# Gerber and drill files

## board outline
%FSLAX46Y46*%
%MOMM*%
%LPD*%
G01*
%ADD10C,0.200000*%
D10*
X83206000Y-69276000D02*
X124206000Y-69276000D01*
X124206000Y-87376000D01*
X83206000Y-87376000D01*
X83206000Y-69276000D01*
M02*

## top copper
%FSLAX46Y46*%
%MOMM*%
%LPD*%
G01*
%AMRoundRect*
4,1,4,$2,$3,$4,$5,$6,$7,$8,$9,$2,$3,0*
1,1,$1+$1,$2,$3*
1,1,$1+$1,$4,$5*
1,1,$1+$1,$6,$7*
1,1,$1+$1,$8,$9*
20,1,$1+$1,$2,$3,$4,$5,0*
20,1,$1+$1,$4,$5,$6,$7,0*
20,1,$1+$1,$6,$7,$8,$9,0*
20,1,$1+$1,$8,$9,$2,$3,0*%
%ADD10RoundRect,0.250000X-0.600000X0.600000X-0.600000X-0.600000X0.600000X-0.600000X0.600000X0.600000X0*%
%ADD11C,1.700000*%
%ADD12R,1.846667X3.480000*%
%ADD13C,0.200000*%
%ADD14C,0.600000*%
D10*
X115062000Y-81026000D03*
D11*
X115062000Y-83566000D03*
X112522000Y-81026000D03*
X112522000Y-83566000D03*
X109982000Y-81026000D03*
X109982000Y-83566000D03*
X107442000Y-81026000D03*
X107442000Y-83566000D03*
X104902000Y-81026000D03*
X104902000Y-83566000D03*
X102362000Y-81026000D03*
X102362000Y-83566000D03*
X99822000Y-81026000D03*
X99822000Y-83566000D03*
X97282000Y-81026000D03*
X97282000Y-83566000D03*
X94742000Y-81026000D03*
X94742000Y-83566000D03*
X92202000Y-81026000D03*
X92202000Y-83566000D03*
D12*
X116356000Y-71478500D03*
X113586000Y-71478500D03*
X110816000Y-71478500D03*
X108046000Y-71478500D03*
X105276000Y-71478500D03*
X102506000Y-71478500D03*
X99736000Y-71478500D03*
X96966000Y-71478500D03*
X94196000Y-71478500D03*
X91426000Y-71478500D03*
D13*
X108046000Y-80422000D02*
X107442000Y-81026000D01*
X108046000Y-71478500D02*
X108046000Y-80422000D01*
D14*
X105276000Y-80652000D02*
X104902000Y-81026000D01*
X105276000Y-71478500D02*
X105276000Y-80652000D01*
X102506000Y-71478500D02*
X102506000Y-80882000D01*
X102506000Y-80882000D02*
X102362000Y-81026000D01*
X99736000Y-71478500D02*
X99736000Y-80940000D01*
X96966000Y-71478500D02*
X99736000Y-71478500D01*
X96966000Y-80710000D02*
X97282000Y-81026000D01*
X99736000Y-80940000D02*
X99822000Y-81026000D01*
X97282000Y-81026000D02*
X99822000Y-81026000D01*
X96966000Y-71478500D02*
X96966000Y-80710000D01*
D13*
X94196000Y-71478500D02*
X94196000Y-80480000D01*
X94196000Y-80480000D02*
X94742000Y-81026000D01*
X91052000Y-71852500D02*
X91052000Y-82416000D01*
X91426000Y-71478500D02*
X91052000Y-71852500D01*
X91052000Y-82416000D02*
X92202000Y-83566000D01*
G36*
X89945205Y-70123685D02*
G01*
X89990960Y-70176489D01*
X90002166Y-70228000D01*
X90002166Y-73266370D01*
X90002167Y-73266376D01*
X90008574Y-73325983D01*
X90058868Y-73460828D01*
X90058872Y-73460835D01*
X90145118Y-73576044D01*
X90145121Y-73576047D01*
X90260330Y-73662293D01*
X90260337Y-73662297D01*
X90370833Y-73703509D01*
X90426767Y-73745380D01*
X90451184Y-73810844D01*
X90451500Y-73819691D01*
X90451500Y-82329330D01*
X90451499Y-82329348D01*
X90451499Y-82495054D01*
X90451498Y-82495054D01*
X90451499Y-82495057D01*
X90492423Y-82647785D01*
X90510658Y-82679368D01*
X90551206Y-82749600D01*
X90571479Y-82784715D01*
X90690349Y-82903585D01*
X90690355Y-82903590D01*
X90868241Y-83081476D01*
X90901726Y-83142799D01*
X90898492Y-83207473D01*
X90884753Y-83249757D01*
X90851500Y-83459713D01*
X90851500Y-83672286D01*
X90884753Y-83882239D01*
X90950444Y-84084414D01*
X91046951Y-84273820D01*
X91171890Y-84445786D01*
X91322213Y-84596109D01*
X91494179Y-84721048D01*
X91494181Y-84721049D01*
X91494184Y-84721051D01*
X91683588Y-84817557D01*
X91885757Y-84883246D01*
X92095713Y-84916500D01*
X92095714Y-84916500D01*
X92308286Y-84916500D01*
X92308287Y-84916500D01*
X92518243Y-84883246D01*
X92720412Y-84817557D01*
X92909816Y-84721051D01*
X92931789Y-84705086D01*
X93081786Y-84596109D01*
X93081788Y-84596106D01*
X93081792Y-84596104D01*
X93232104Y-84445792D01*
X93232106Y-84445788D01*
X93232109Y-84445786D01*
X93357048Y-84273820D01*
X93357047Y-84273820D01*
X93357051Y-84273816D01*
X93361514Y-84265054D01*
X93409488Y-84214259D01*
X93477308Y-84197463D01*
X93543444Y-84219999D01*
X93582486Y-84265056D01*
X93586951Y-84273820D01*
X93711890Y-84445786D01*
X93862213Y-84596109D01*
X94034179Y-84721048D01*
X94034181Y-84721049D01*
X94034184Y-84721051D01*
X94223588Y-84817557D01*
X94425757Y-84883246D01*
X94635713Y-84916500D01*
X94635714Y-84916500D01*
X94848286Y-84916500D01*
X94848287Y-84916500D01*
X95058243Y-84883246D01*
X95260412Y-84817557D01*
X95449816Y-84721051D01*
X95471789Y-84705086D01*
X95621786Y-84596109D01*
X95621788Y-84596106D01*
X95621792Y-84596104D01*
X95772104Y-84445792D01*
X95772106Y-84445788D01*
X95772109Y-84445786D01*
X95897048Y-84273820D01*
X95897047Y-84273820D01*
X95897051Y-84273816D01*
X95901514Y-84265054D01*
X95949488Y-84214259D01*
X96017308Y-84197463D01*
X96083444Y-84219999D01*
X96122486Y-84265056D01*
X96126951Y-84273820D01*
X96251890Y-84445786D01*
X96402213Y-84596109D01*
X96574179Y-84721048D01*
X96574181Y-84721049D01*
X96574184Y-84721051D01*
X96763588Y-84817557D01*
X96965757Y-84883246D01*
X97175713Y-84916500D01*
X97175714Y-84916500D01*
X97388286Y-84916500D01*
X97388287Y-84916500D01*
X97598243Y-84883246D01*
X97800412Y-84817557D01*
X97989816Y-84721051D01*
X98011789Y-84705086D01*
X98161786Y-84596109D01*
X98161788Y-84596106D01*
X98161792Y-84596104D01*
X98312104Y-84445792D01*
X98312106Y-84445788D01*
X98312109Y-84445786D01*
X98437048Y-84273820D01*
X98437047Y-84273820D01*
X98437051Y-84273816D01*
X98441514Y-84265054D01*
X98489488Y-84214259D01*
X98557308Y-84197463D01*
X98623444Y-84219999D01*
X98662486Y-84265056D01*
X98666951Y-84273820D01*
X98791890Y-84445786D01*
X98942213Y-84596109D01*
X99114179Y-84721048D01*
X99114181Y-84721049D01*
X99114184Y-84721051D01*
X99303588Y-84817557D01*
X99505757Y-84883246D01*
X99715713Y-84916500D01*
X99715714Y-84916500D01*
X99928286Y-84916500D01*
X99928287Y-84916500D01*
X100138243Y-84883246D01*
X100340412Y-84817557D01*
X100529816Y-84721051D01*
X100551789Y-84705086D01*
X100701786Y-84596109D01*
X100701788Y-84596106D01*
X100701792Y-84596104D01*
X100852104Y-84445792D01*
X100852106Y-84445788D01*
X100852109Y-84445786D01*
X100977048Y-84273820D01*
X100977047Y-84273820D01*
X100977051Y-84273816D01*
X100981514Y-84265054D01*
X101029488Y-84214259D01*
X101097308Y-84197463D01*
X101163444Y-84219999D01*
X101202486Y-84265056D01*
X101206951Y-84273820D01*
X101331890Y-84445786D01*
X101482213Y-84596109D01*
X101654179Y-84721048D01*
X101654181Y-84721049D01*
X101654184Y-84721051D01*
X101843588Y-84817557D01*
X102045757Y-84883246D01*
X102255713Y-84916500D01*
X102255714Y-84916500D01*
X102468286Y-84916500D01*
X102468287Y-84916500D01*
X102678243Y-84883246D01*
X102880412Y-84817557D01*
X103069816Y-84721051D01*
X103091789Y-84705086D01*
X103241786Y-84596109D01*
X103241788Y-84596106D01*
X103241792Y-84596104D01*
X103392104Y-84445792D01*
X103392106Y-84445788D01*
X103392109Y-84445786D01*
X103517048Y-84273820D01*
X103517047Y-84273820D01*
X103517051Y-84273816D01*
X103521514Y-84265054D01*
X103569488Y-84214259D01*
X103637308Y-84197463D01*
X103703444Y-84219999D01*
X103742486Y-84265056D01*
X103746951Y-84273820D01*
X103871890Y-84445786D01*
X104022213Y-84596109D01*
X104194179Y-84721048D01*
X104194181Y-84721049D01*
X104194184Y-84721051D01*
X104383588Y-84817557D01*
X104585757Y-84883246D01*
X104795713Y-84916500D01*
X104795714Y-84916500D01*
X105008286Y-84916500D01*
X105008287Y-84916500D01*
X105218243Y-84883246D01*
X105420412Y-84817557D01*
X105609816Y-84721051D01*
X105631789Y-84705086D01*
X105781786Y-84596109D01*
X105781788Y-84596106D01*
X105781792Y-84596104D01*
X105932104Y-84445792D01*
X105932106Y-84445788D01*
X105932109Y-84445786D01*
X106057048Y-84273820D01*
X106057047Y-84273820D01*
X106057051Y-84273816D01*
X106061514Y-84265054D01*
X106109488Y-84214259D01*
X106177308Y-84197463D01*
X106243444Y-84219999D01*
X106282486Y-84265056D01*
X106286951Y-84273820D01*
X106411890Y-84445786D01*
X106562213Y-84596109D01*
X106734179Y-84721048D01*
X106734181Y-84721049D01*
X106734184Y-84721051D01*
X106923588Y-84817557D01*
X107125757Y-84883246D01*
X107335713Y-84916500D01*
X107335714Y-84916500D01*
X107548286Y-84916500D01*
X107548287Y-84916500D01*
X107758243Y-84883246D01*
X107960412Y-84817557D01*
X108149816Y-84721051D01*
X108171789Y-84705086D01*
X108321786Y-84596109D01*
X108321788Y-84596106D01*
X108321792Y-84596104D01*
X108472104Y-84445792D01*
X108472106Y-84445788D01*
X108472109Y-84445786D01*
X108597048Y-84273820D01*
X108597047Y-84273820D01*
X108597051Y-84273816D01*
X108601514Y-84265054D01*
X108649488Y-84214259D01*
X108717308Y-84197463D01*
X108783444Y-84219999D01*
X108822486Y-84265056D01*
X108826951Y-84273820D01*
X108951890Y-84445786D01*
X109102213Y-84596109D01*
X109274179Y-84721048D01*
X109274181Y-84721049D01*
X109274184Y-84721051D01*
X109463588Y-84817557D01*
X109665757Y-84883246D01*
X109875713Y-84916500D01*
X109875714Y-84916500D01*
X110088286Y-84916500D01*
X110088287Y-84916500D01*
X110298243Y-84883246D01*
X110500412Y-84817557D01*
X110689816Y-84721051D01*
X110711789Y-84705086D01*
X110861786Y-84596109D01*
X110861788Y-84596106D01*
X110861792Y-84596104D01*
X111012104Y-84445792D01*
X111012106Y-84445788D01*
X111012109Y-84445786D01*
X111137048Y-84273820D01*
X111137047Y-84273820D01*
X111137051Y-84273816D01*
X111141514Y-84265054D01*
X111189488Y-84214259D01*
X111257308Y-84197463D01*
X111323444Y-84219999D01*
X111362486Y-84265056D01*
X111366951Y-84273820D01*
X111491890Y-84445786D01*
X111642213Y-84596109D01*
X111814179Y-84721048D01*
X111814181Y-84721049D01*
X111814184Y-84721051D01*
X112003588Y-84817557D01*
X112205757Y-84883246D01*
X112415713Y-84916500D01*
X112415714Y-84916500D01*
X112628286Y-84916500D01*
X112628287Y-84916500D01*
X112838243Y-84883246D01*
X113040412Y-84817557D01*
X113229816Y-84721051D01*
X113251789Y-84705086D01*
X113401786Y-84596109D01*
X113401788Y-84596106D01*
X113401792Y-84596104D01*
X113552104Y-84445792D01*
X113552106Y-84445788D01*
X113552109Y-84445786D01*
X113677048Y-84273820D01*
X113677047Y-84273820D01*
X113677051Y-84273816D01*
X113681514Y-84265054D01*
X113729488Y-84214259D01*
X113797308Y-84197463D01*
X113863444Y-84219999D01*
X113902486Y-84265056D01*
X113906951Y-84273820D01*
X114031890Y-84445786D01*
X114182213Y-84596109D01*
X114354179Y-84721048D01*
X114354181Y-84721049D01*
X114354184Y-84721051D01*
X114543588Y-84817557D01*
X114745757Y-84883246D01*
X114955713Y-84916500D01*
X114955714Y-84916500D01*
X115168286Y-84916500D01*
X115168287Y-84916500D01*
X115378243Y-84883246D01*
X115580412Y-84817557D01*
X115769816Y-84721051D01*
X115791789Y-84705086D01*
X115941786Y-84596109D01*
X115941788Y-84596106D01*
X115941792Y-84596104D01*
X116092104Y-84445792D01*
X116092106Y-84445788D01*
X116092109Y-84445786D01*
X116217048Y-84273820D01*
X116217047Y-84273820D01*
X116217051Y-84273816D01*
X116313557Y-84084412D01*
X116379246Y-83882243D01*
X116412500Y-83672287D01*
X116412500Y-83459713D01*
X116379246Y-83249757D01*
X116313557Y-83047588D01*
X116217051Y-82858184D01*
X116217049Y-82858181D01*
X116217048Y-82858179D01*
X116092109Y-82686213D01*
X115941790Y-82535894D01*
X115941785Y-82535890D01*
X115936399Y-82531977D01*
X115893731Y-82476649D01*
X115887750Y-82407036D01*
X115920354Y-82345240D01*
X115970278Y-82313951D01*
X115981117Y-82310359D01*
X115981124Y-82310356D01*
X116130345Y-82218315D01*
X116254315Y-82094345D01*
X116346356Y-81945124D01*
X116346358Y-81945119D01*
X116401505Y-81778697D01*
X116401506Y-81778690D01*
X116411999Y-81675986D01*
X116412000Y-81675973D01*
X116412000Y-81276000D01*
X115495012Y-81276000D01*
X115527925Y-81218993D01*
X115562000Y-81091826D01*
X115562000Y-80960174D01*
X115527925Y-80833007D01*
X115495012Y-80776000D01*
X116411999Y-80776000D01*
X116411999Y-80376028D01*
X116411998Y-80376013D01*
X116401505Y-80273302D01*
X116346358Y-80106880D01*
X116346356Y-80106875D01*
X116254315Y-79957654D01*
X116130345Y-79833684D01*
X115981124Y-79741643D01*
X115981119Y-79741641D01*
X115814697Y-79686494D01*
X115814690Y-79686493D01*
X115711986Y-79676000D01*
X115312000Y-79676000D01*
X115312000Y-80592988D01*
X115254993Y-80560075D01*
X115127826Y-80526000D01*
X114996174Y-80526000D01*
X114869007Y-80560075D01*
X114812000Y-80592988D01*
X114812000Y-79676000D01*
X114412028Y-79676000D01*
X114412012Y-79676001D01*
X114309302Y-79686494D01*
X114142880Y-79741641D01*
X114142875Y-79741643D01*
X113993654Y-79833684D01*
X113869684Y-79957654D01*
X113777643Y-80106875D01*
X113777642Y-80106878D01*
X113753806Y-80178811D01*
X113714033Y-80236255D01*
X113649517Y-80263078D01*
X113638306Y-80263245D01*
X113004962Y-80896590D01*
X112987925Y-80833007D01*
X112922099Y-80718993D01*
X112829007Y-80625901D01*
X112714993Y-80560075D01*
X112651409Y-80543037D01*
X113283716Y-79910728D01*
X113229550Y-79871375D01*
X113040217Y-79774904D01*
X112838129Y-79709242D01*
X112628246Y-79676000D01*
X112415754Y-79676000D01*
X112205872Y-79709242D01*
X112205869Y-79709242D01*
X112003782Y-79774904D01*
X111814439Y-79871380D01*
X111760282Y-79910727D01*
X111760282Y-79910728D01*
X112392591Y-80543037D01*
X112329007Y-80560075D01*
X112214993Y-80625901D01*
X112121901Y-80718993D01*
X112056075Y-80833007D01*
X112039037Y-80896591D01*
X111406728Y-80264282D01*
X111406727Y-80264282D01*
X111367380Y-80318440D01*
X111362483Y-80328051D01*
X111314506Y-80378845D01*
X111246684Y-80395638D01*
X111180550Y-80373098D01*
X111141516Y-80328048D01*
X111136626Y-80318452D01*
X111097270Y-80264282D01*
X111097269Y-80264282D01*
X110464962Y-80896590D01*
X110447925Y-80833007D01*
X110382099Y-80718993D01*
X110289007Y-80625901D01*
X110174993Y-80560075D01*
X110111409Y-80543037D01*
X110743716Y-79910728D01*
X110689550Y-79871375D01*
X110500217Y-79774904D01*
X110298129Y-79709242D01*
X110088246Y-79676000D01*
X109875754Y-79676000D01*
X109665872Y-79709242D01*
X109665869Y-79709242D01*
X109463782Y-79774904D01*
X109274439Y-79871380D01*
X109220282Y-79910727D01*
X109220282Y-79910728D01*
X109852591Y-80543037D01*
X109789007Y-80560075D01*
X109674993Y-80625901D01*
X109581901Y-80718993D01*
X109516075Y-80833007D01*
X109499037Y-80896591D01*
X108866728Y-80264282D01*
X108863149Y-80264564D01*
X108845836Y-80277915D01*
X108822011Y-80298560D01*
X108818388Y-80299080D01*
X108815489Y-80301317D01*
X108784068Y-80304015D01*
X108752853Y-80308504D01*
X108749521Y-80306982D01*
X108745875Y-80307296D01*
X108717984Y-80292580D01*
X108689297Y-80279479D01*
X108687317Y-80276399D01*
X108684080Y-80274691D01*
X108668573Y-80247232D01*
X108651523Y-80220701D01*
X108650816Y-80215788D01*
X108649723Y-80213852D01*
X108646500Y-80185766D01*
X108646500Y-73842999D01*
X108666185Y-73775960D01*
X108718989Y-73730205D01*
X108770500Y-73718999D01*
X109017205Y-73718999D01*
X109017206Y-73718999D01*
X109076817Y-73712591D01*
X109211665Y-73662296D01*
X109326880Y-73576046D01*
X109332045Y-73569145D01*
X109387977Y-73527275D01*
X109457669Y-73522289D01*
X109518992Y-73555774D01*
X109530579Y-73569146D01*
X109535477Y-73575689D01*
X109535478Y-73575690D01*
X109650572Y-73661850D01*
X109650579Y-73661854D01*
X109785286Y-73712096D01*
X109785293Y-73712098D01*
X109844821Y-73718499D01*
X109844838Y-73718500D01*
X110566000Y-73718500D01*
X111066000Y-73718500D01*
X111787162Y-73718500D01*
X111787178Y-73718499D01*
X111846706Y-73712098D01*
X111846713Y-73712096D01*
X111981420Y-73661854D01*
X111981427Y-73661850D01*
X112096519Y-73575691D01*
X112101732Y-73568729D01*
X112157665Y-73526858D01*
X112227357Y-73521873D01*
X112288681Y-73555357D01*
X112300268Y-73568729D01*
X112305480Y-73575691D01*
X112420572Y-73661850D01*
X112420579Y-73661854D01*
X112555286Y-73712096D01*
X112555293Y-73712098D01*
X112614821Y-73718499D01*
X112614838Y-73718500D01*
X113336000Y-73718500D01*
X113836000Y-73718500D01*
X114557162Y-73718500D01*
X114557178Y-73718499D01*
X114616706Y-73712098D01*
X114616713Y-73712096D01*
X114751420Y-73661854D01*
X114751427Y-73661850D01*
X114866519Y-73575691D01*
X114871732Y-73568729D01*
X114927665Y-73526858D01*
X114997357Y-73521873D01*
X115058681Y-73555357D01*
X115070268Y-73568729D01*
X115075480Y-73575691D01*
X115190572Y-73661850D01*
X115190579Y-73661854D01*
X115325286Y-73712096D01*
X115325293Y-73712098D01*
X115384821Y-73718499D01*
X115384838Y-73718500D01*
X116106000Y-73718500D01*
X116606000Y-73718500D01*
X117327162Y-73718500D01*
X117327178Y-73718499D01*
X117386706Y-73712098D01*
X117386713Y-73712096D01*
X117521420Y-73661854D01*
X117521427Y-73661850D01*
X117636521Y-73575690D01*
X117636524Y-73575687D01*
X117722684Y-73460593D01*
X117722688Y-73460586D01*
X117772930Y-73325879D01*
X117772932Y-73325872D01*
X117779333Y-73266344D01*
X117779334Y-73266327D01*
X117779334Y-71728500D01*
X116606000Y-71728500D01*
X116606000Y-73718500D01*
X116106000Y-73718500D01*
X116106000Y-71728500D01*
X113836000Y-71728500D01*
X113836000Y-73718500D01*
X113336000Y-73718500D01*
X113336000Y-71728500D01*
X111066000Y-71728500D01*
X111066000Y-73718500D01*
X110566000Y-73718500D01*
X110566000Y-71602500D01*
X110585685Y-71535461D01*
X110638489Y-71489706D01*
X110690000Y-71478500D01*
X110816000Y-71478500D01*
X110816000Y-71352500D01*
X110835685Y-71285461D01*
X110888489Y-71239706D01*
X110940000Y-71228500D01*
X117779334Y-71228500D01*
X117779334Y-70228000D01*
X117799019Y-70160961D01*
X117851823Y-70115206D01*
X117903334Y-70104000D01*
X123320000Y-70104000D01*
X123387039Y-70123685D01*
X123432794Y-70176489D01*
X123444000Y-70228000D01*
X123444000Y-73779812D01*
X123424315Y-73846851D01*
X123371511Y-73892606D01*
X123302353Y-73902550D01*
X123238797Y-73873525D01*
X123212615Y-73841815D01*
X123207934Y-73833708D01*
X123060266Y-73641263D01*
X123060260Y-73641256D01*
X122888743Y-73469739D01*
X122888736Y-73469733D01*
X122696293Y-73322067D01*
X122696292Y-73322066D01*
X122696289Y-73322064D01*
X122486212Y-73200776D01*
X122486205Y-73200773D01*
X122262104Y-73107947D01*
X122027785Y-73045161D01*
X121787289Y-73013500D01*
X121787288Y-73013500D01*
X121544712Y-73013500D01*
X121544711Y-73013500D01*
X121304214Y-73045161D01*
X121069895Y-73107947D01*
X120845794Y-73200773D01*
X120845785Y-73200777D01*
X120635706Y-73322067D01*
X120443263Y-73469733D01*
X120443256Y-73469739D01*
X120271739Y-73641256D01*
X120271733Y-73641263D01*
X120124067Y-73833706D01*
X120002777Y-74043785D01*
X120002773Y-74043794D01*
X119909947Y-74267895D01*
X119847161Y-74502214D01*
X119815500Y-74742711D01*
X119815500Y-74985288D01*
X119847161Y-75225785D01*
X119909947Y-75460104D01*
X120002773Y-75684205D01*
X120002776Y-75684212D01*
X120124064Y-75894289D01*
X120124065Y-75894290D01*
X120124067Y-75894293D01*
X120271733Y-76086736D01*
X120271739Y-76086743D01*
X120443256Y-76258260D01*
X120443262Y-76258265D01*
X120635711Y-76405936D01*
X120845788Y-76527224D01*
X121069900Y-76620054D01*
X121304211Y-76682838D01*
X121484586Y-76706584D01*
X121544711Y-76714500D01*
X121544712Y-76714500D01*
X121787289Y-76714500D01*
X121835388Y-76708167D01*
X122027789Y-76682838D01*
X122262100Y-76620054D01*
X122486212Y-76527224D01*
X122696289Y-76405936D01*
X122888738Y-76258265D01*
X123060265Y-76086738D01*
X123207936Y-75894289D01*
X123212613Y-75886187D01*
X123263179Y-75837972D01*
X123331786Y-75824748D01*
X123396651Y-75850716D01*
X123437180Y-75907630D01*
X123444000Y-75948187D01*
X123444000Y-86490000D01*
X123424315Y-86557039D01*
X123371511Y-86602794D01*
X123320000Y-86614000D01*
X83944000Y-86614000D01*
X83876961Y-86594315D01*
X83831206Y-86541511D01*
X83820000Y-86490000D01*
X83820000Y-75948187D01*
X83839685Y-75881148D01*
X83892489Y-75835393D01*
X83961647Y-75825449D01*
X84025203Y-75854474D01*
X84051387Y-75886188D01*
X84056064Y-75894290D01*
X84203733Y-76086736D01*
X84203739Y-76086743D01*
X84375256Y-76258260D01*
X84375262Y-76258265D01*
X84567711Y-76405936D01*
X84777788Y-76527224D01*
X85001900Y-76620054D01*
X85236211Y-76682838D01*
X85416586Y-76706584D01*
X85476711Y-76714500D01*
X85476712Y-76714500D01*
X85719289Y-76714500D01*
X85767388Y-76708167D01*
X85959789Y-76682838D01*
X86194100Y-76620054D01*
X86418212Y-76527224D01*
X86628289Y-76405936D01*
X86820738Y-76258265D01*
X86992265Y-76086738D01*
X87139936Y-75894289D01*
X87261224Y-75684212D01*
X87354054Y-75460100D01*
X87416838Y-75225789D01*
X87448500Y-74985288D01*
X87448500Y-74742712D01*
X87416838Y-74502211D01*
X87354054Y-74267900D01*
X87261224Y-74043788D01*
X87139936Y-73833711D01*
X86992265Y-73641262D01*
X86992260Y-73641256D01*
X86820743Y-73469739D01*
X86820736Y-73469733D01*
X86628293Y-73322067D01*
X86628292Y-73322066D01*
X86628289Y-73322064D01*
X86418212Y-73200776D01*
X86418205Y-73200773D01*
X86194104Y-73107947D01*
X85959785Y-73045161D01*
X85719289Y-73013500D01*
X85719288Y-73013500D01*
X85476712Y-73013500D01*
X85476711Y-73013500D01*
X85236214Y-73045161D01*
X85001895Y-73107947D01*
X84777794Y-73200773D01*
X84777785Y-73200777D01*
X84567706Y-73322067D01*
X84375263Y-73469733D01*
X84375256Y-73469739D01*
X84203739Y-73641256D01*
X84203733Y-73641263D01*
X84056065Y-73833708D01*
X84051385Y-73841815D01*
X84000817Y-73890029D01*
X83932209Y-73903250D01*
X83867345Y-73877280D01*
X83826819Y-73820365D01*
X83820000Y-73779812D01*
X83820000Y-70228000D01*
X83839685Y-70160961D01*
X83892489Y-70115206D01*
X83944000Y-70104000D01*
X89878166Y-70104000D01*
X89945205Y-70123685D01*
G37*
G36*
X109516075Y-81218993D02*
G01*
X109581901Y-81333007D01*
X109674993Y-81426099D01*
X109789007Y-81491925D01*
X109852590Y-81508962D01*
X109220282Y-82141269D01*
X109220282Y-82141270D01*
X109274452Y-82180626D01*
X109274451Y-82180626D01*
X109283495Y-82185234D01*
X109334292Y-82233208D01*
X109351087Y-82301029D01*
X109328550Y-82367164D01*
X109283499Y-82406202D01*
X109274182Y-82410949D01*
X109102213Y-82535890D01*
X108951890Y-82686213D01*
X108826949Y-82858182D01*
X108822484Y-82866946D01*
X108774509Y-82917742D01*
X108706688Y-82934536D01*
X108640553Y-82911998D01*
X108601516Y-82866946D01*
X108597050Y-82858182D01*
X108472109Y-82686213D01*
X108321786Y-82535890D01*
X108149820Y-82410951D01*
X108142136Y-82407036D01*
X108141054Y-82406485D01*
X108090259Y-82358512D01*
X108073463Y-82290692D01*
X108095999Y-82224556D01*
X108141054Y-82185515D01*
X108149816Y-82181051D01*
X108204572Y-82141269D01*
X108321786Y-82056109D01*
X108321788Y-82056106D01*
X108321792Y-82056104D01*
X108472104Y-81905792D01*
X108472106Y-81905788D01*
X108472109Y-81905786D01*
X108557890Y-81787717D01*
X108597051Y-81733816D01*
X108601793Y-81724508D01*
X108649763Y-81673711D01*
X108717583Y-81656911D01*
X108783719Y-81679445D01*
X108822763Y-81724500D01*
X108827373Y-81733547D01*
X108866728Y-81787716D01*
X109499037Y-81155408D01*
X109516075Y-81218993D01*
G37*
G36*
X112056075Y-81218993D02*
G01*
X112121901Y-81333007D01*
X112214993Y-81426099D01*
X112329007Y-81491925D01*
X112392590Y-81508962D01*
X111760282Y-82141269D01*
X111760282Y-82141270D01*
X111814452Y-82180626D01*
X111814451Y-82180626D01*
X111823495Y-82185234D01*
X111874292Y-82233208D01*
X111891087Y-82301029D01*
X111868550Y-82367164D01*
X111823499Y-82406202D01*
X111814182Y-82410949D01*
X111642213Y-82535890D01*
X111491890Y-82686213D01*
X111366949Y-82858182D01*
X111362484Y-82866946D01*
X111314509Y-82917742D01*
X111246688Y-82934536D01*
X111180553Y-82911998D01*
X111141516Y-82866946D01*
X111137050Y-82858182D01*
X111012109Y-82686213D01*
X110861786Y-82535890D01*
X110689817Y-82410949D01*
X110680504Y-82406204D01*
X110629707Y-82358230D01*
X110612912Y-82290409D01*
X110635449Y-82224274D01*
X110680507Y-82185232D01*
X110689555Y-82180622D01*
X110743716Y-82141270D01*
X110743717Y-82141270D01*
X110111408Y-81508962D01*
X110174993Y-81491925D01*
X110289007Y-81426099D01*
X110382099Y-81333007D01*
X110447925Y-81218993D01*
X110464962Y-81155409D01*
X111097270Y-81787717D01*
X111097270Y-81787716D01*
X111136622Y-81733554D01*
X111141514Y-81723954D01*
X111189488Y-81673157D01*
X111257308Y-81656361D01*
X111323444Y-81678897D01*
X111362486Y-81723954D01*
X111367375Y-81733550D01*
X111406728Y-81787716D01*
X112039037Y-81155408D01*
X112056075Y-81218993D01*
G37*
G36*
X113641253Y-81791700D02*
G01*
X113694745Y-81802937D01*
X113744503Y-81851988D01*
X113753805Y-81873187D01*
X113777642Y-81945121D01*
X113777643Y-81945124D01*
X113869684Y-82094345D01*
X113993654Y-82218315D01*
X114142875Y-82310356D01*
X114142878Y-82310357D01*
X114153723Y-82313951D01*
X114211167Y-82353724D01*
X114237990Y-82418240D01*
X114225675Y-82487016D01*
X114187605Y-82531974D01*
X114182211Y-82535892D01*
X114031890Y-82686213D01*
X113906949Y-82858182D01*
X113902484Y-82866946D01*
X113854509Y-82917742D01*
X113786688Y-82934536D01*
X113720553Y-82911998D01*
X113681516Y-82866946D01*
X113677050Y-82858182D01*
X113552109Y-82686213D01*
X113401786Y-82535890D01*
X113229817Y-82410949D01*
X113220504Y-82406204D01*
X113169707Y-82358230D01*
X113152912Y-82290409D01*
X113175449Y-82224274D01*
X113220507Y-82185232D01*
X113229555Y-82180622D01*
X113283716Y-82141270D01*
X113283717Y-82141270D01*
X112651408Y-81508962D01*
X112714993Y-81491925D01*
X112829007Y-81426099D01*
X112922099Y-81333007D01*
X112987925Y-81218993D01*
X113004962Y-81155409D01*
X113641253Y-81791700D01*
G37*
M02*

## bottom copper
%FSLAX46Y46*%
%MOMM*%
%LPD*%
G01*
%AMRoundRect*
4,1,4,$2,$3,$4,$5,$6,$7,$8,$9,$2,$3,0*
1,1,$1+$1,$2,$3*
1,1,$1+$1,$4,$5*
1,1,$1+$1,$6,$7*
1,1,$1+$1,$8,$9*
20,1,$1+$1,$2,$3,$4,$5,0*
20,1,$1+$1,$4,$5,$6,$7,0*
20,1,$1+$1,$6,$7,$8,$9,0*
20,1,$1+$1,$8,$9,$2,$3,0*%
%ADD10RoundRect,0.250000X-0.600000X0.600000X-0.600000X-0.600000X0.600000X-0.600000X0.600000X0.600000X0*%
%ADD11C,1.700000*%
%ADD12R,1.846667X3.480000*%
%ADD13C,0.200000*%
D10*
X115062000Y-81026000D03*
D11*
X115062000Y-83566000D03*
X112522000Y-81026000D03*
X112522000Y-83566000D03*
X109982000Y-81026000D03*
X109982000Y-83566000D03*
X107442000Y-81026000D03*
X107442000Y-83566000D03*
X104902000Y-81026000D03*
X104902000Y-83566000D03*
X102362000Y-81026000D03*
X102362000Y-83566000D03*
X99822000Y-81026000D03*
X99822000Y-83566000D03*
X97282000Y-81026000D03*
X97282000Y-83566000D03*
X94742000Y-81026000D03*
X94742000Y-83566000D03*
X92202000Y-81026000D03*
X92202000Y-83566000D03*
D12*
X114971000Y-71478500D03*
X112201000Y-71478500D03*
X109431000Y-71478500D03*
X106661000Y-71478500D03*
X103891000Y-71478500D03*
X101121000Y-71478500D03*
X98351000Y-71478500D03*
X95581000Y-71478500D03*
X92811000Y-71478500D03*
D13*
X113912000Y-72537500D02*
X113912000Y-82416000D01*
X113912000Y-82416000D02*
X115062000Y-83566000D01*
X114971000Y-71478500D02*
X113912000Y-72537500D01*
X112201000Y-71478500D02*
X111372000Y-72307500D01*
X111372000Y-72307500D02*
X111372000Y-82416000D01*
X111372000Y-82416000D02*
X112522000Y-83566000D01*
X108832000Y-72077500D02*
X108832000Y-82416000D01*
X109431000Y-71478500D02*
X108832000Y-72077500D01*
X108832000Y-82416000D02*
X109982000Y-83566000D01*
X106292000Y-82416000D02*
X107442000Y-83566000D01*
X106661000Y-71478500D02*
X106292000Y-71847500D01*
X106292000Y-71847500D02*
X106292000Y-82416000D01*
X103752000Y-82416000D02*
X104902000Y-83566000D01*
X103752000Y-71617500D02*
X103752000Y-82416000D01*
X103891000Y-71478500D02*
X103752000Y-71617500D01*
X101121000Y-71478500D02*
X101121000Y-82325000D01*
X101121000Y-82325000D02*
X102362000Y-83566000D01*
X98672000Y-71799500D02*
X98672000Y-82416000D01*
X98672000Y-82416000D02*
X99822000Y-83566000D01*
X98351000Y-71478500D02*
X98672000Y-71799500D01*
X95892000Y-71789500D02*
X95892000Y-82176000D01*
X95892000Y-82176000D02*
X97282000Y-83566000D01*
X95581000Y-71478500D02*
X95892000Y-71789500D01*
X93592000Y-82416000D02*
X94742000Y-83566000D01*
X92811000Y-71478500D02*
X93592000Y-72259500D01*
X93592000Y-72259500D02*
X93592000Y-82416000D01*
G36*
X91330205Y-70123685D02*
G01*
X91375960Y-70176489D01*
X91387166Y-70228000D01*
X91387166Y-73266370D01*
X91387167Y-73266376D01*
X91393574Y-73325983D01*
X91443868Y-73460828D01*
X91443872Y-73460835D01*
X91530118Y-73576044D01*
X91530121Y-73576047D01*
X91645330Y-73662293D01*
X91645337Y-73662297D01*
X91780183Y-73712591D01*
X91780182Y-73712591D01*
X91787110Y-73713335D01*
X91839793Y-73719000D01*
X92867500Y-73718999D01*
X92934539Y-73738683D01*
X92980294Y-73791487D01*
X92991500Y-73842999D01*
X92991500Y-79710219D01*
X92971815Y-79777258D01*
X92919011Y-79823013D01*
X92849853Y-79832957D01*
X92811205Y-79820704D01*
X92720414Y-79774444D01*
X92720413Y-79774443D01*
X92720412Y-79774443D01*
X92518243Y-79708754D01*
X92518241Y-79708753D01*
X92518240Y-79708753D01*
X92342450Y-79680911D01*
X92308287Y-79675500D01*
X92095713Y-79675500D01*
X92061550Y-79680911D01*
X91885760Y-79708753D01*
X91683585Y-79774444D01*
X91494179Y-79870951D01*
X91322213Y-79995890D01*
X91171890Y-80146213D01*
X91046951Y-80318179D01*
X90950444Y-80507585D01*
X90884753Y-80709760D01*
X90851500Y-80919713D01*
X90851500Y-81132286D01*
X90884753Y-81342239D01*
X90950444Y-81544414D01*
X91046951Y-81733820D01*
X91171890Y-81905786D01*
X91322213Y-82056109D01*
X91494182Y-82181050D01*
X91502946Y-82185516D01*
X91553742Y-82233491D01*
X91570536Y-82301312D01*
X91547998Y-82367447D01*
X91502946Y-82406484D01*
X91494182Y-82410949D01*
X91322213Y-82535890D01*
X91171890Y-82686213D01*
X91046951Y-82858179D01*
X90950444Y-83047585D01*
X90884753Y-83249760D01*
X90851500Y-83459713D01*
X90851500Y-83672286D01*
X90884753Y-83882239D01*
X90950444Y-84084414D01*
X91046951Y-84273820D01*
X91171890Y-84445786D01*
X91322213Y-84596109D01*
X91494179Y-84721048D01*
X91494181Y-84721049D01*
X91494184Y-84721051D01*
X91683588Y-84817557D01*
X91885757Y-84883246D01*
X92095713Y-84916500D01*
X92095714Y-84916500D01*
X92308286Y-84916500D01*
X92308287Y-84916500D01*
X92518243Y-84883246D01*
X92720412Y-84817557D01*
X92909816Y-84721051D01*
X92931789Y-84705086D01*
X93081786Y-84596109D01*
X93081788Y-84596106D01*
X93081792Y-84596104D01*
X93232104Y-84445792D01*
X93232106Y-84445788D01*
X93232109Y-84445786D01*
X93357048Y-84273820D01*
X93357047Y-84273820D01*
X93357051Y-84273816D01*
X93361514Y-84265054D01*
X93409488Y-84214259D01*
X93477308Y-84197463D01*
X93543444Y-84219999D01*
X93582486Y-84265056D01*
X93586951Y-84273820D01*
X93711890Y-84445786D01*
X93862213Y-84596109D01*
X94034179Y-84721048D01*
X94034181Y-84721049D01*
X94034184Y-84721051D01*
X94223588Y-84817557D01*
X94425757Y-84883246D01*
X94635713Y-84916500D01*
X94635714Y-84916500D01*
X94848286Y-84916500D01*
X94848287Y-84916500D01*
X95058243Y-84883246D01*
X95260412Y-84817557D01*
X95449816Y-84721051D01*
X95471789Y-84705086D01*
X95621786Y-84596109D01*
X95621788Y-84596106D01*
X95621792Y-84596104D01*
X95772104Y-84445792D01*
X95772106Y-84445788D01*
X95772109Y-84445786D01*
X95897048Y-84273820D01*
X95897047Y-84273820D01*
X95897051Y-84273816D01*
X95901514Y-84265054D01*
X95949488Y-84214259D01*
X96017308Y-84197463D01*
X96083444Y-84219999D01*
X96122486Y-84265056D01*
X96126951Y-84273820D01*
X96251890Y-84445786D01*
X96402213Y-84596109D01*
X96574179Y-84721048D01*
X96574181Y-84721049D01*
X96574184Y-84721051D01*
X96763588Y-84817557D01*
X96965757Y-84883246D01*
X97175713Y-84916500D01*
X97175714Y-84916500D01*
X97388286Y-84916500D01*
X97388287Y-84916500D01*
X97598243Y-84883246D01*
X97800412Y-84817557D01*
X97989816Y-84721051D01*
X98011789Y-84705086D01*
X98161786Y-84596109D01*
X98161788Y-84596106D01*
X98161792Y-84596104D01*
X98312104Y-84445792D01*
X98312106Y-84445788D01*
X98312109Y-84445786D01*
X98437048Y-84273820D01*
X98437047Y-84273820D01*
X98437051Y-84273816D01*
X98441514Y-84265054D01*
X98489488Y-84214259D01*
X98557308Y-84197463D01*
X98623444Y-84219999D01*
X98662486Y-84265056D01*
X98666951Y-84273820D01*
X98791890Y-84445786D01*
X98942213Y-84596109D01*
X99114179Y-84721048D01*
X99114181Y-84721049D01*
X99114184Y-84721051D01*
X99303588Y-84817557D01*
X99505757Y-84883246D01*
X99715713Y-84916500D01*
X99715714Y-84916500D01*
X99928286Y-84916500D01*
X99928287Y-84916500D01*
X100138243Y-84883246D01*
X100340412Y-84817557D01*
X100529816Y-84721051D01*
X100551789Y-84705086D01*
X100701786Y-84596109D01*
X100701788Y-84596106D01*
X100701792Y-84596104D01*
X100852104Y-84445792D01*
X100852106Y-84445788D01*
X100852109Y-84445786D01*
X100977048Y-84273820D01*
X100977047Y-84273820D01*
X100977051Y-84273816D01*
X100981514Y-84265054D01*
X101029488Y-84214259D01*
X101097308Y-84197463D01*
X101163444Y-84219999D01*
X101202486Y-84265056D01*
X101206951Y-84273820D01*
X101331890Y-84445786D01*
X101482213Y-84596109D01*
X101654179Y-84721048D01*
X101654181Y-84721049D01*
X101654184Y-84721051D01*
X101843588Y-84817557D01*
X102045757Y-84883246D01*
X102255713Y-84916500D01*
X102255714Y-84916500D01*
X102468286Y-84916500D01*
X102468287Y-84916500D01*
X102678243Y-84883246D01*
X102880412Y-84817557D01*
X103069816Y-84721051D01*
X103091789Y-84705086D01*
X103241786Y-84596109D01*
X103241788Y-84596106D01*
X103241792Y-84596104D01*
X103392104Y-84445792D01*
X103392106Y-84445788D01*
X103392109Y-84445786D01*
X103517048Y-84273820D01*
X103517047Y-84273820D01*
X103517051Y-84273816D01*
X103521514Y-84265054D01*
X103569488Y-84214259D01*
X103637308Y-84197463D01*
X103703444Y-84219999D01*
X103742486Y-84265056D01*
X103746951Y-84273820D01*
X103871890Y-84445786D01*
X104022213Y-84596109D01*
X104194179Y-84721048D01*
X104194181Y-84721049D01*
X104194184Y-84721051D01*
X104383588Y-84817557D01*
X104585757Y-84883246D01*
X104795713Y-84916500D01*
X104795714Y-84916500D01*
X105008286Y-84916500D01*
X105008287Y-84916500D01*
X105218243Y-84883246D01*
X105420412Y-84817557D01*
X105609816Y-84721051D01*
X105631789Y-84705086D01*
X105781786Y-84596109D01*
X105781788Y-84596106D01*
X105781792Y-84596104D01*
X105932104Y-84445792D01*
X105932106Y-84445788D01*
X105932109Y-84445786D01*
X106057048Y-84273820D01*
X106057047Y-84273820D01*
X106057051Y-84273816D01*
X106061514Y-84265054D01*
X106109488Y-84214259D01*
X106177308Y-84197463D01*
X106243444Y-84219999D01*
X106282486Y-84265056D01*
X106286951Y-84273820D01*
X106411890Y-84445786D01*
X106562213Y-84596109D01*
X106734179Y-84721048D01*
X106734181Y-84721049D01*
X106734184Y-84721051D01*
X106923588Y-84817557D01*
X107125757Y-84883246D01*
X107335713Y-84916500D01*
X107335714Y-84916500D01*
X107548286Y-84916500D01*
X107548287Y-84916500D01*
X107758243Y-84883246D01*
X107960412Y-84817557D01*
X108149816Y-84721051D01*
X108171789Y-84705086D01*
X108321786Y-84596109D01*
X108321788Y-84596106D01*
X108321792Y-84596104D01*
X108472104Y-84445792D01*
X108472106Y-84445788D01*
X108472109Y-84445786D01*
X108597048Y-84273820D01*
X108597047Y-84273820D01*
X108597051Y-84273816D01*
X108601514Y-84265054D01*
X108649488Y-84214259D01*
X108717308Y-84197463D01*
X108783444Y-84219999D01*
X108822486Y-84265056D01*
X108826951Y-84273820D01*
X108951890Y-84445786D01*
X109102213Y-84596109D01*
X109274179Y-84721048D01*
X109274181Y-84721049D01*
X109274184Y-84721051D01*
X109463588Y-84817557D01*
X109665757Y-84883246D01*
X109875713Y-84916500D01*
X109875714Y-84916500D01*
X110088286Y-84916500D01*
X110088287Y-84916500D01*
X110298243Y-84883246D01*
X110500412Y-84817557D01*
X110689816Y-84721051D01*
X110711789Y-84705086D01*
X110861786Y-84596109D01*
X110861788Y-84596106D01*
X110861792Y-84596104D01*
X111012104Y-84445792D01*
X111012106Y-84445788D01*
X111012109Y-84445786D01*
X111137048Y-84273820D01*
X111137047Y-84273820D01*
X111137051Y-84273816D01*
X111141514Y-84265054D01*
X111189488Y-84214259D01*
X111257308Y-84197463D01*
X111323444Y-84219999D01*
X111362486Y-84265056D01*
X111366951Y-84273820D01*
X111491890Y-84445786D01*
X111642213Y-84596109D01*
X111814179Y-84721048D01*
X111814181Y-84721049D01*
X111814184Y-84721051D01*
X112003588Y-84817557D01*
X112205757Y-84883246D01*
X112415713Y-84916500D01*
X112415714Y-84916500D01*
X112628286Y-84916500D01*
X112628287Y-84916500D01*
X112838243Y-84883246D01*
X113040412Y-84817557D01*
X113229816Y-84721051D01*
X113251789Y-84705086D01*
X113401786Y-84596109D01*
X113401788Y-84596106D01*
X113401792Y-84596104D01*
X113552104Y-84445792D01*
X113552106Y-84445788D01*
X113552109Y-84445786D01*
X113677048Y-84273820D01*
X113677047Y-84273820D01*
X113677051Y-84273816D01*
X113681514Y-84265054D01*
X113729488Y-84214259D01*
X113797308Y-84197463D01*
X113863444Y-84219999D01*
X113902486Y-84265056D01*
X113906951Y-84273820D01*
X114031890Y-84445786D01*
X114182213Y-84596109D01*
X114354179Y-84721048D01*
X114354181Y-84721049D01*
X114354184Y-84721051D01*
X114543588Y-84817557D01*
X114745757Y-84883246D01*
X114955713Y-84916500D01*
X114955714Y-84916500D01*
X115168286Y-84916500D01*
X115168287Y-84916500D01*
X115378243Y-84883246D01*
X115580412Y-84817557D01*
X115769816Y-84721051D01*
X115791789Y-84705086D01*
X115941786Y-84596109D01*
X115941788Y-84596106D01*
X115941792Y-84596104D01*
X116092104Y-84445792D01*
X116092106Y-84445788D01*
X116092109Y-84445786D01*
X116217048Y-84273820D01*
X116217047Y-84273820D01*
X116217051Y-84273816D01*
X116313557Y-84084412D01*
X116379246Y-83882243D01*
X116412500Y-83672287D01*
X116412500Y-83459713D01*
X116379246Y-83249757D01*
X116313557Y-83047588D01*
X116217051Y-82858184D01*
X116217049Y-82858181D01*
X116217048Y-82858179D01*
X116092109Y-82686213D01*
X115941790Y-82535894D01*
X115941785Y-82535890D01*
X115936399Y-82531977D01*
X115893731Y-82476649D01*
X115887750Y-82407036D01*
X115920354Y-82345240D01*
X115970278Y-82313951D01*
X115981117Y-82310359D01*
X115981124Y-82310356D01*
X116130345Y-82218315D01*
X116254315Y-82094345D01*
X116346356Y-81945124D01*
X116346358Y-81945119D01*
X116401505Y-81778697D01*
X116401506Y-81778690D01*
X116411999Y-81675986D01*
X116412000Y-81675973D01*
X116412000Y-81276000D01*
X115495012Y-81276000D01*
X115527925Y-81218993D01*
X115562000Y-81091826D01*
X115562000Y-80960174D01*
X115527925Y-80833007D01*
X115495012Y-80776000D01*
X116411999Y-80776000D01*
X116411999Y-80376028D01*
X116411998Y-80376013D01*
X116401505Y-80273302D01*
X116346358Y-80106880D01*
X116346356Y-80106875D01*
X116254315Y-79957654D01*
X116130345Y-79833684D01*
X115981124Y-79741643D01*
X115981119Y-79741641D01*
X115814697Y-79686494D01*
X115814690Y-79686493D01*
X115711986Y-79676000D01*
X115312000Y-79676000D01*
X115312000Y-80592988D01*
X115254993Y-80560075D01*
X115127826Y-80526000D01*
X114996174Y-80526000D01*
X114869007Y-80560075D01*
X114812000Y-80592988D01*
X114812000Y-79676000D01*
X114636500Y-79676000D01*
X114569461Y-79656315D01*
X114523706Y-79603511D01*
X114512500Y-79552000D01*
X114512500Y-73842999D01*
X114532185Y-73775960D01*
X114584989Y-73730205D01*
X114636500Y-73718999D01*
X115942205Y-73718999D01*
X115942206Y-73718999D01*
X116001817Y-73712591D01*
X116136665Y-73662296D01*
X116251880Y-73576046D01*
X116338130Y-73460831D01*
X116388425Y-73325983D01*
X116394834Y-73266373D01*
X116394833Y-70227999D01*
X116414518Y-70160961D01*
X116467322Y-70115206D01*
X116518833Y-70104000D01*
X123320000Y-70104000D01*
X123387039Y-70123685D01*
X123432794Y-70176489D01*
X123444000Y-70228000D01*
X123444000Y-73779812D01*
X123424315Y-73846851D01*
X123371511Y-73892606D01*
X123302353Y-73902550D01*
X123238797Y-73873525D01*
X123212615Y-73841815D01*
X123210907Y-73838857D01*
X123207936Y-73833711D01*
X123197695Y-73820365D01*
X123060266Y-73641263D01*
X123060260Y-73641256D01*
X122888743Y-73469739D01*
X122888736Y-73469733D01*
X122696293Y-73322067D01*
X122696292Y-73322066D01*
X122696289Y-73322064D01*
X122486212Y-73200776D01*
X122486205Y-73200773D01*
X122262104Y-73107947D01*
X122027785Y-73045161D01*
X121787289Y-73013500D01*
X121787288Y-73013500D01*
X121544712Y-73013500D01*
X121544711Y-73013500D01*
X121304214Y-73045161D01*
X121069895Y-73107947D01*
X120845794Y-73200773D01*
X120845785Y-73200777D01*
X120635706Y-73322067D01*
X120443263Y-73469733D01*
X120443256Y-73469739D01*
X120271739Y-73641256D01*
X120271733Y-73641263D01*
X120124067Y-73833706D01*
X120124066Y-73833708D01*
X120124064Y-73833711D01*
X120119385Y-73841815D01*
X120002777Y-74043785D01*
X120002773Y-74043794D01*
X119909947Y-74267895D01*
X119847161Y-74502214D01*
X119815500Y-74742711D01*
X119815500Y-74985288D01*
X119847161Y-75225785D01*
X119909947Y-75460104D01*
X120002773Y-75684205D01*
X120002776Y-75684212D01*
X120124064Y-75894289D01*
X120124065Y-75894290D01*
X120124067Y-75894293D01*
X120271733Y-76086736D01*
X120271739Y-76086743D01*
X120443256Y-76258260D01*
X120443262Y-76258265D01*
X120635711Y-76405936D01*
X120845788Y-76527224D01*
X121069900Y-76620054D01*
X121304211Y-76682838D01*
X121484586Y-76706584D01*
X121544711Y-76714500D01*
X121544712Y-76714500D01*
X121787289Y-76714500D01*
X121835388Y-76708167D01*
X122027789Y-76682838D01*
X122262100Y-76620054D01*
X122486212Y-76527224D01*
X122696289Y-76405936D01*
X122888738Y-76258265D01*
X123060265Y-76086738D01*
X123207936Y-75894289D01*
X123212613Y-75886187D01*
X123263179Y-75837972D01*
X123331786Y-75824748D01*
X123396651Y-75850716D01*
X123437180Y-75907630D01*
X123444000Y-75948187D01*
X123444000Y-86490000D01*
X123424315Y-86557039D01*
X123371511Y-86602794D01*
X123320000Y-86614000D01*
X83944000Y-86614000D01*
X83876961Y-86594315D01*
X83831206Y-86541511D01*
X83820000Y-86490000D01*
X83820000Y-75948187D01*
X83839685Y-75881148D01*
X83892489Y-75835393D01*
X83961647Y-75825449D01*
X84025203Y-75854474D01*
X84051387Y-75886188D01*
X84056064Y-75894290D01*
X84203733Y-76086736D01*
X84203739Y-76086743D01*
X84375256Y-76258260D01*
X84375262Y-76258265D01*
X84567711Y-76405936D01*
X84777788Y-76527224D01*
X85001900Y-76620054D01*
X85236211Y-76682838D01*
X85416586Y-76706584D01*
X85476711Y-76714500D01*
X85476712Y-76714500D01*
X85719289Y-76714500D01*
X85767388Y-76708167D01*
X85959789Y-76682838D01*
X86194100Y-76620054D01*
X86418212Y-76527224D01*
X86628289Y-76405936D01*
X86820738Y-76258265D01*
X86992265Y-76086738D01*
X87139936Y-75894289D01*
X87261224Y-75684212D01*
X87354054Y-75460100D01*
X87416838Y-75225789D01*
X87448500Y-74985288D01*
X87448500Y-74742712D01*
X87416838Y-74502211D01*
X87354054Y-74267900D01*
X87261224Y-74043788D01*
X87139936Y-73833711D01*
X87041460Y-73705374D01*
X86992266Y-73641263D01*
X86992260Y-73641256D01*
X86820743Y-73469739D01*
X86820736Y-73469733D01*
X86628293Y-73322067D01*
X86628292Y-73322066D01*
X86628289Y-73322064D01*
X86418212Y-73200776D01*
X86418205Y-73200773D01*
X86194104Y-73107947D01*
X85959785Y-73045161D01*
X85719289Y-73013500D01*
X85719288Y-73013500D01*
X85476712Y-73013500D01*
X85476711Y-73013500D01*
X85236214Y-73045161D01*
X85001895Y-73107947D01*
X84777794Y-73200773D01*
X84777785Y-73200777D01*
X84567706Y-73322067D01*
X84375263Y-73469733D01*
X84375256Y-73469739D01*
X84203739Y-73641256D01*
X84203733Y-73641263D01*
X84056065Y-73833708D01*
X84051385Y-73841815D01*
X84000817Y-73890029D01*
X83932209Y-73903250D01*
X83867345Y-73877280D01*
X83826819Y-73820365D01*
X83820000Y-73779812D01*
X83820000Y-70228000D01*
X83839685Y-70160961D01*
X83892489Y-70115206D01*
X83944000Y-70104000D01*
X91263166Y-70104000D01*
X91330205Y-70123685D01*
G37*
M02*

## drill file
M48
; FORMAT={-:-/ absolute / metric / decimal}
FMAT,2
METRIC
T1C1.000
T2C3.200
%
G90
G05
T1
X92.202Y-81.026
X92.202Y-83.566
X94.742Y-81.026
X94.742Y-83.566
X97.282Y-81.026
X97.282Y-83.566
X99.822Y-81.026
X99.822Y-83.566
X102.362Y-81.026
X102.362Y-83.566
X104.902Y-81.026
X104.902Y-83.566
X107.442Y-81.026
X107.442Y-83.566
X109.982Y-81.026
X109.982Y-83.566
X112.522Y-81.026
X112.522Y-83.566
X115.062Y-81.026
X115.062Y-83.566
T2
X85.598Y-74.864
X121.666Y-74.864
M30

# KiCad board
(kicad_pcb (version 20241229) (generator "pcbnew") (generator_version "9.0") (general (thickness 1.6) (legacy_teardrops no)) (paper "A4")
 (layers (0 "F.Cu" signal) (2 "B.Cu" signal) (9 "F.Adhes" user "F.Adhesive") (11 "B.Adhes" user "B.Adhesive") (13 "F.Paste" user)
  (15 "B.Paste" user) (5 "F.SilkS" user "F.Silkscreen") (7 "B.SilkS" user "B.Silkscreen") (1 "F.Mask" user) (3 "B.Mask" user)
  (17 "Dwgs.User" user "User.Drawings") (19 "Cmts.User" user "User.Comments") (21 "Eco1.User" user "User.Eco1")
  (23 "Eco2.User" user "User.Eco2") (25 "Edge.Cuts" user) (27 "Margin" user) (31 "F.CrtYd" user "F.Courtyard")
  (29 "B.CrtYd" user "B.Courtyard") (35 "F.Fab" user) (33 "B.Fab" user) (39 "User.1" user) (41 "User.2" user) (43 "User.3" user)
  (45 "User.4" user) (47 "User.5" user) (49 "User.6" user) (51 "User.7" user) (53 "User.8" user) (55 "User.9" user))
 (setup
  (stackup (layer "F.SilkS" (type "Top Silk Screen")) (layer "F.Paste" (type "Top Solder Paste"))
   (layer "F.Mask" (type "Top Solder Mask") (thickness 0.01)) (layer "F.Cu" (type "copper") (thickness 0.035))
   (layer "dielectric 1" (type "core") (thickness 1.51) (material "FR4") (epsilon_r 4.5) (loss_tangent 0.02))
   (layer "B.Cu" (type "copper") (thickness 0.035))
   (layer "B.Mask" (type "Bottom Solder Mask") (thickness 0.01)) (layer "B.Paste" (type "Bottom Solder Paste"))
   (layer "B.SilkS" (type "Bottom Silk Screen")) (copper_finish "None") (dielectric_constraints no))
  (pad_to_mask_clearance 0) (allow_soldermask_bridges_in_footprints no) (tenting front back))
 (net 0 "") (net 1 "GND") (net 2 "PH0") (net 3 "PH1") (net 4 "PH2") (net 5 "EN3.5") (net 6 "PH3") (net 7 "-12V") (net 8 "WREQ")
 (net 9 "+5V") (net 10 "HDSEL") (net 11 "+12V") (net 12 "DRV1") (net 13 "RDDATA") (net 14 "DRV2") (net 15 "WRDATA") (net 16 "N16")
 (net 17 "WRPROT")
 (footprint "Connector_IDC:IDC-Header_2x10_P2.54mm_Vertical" (layer "F.Cu") (at 115.062 81.026 -90)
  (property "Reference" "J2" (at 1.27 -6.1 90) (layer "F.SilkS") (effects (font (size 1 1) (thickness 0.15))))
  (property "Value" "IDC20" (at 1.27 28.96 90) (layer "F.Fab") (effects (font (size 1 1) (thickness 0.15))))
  (pad "1" thru_hole roundrect (at 0 0 270) (size 1.7 1.7) (drill 1) (layers "*.Cu" "*.Mask") (remove_unused_layers no)
   (roundrect_rratio 0.147059) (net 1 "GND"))
  (pad "2" thru_hole circle (at 2.54 0 270) (size 1.7 1.7) (drill 1) (layers "*.Cu" "*.Mask") (remove_unused_layers no) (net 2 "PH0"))
  (pad "3" thru_hole circle (at 0 2.54 270) (size 1.7 1.7) (drill 1) (layers "*.Cu" "*.Mask") (remove_unused_layers no) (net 1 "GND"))
  (pad "4" thru_hole circle (at 2.54 2.54 270) (size 1.7 1.7) (drill 1) (layers "*.Cu" "*.Mask") (remove_unused_layers no) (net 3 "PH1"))
  (pad "5" thru_hole circle (at 0 5.08 270) (size 1.7 1.7) (drill 1) (layers "*.Cu" "*.Mask") (remove_unused_layers no) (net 1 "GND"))
  (pad "6" thru_hole circle (at 2.54 5.08 270) (size 1.7 1.7) (drill 1) (layers "*.Cu" "*.Mask") (remove_unused_layers no) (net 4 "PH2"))
  (pad "7" thru_hole circle (at 0 7.62 270) (size 1.7 1.7) (drill 1) (layers "*.Cu" "*.Mask") (remove_unused_layers no) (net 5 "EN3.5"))
  (pad "8" thru_hole circle (at 2.54 7.62 270) (size 1.7 1.7) (drill 1) (layers "*.Cu" "*.Mask") (remove_unused_layers no) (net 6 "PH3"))
  (pad "9" thru_hole circle (at 0 10.16 270) (size 1.7 1.7) (drill 1) (layers "*.Cu" "*.Mask") (remove_unused_layers no) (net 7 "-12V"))
  (pad "10" thru_hole circle (at 2.54 10.16 270) (size 1.7 1.7) (drill 1) (layers "*.Cu" "*.Mask") (remove_unused_layers no) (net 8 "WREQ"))
  (pad "11" thru_hole circle (at 0 12.7 270) (size 1.7 1.7) (drill 1) (layers "*.Cu" "*.Mask") (remove_unused_layers no) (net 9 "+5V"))
  (pad "12" thru_hole circle (at 2.54 12.7 270) (size 1.7 1.7) (drill 1) (layers "*.Cu" "*.Mask") (remove_unused_layers no) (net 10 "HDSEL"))
  (pad "13" thru_hole circle (at 0 15.24 270) (size 1.7 1.7) (drill 1) (layers "*.Cu" "*.Mask") (remove_unused_layers no) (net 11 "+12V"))
  (pad "14" thru_hole circle (at 2.54 15.24 270) (size 1.7 1.7) (drill 1) (layers "*.Cu" "*.Mask") (remove_unused_layers no) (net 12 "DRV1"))
  (pad "15" thru_hole circle (at 0 17.78 270) (size 1.7 1.7) (drill 1) (layers "*.Cu" "*.Mask") (remove_unused_layers no) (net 11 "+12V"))
  (pad "16" thru_hole circle (at 2.54 17.78 270) (size 1.7 1.7) (drill 1) (layers "*.Cu" "*.Mask") (remove_unused_layers no)
   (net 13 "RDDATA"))
  (pad "17" thru_hole circle (at 0 20.32 270) (size 1.7 1.7) (drill 1) (layers "*.Cu" "*.Mask") (remove_unused_layers no) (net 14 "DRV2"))
  (pad "18" thru_hole circle (at 2.54 20.32 270) (size 1.7 1.7) (drill 1) (layers "*.Cu" "*.Mask") (remove_unused_layers no)
   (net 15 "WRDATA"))
  (pad "19" thru_hole circle (at 0 22.86 270) (size 1.7 1.7) (drill 1) (layers "*.Cu" "*.Mask") (remove_unused_layers no) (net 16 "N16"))
  (pad "20" thru_hole circle (at 2.54 22.86 270) (size 1.7 1.7) (drill 1) (layers "*.Cu" "*.Mask") (remove_unused_layers no)
   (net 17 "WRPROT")))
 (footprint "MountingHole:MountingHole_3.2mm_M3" (layer "F.Cu") (at 121.666 74.864)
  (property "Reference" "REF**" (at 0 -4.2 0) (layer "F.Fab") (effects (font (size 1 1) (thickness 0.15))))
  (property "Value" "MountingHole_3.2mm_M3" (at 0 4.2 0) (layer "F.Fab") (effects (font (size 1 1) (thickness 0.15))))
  (pad "" np_thru_hole circle (at 0 0) (size 3.2 3.2) (drill 3.2) (layers "*.Cu" "*.Mask")))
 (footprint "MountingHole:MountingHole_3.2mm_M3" (layer "F.Cu") (at 85.598 74.864)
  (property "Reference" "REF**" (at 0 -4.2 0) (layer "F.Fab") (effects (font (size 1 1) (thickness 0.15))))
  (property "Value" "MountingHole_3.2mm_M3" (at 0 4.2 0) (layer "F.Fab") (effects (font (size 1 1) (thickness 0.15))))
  (pad "" np_thru_hole circle (at 0 0) (size 3.2 3.2) (drill 3.2) (layers "*.Cu" "*.Mask")))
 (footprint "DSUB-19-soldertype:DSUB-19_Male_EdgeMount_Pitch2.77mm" (layer "F.Cu") (at 103.886 71.4785 180)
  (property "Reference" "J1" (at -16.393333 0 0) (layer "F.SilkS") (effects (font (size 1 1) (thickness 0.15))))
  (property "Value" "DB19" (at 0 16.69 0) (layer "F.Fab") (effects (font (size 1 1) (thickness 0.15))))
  (pad "1" smd rect (at -12.47 0 180) (size 1.846667 3.48) (layers "F.Cu" "F.Mask" "F.Paste") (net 1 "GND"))
  (pad "2" smd rect (at -9.7 0 180) (size 1.846667 3.48) (layers "F.Cu" "F.Mask" "F.Paste") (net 1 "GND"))
  (pad "3" smd rect (at -6.93 0 180) (size 1.846667 3.48) (layers "F.Cu" "F.Mask" "F.Paste") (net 1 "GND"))
  (pad "4" smd rect (at -4.16 0 180) (size 1.846667 3.48) (layers "F.Cu" "F.Mask" "F.Paste") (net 5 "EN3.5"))
  (pad "5" smd rect (at -1.39 0 180) (size 1.846667 3.48) (layers "F.Cu" "F.Mask" "F.Paste") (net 7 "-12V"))
  (pad "6" smd rect (at 1.38 0 180) (size 1.846667 3.48) (layers "F.Cu" "F.Mask" "F.Paste") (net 9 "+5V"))
  (pad "7" smd rect (at 4.15 0 180) (size 1.846667 3.48) (layers "F.Cu" "F.Mask" "F.Paste") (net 11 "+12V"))
  (pad "8" smd rect (at 6.92 0 180) (size 1.846667 3.48) (layers "F.Cu" "F.Mask" "F.Paste") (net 11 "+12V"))
  (pad "9" smd rect (at 9.69 0 180) (size 1.846667 3.48) (layers "F.Cu" "F.Mask" "F.Paste") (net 14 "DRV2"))
  (pad "10" smd rect (at 12.46 0 180) (size 1.846667 3.48) (layers "F.Cu" "F.Mask" "F.Paste") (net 17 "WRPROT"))
  (pad "11" smd rect (at -11.085 0 180) (size 1.846667 3.48) (layers "B.Cu" "B.Mask" "B.Paste") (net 2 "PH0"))
  (pad "12" smd rect (at -8.315 0 180) (size 1.846667 3.48) (layers "B.Cu" "B.Mask" "B.Paste") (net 3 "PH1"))
  (pad "13" smd rect (at -5.545 0 180) (size 1.846667 3.48) (layers "B.Cu" "B.Mask" "B.Paste") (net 4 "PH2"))
  (pad "14" smd rect (at -2.775 0 180) (size 1.846667 3.48) (layers "B.Cu" "B.Mask" "B.Paste") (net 6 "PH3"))
  (pad "15" smd rect (at -0.005 0 180) (size 1.846667 3.48) (layers "B.Cu" "B.Mask" "B.Paste") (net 8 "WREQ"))
  (pad "16" smd rect (at 2.765 0 180) (size 1.846667 3.48) (layers "B.Cu" "B.Mask" "B.Paste") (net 10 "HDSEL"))
  (pad "17" smd rect (at 5.535 0 180) (size 1.846667 3.48) (layers "B.Cu" "B.Mask" "B.Paste") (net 12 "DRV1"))
  (pad "18" smd rect (at 8.305 0 180) (size 1.846667 3.48) (layers "B.Cu" "B.Mask" "B.Paste") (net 13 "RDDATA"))
  (pad "19" smd rect (at 11.075 0 180) (size 1.846667 3.48) (layers "B.Cu" "B.Mask" "B.Paste") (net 15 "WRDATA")))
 (gr_rect (start 83.206 69.276) (end 124.206 87.376) (stroke (width 0.2) (type solid)) (fill no) (layer "Edge.Cuts"))
 (segment (start 108.046 80.422) (end 107.442 81.026) (width 0.2) (layer "F.Cu") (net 5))
 (segment (start 108.046 71.4785) (end 108.046 80.422) (width 0.2) (layer "F.Cu") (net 5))
 (segment (start 105.276 80.652) (end 104.902 81.026) (width 0.6) (layer "F.Cu") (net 7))
 (segment (start 105.276 71.4785) (end 105.276 80.652) (width 0.6) (layer "F.Cu") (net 7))
 (segment (start 102.506 71.4785) (end 102.506 80.882) (width 0.6) (layer "F.Cu") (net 9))
 (segment (start 102.506 80.882) (end 102.362 81.026) (width 0.6) (layer "F.Cu") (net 9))
 (segment (start 99.736 71.4785) (end 99.736 80.94) (width 0.6) (layer "F.Cu") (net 11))
 (segment (start 96.966 71.4785) (end 99.736 71.4785) (width 0.6) (layer "F.Cu") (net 11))
 (segment (start 96.966 80.71) (end 97.282 81.026) (width 0.6) (layer "F.Cu") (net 11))
 (segment (start 99.736 80.94) (end 99.822 81.026) (width 0.6) (layer "F.Cu") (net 11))
 (segment (start 97.282 81.026) (end 99.822 81.026) (width 0.6) (layer "F.Cu") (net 11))
 (segment (start 96.966 71.4785) (end 96.966 80.71) (width 0.6) (layer "F.Cu") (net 11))
 (segment (start 94.196 71.4785) (end 94.196 80.48) (width 0.2) (layer "F.Cu") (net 14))
 (segment (start 94.196 80.48) (end 94.742 81.026) (width 0.2) (layer "F.Cu") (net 14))
 (segment (start 91.052 71.8525) (end 91.052 82.416) (width 0.2) (layer "F.Cu") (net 17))
 (segment (start 91.426 71.4785) (end 91.052 71.8525) (width 0.2) (layer "F.Cu") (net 17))
 (segment (start 91.052 82.416) (end 92.202 83.566) (width 0.2) (layer "F.Cu") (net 17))
 (segment (start 113.912 72.5375) (end 113.912 82.416) (width 0.2) (layer "B.Cu") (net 2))
 (segment (start 113.912 82.416) (end 115.062 83.566) (width 0.2) (layer "B.Cu") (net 2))
 (segment (start 114.971 71.4785) (end 113.912 72.5375) (width 0.2) (layer "B.Cu") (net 2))
 (segment (start 112.201 71.4785) (end 111.372 72.3075) (width 0.2) (layer "B.Cu") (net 3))
 (segment (start 111.372 72.3075) (end 111.372 82.416) (width 0.2) (layer "B.Cu") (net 3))
 (segment (start 111.372 82.416) (end 112.522 83.566) (width 0.2) (layer "B.Cu") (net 3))
 (segment (start 108.832 72.0775) (end 108.832 82.416) (width 0.2) (layer "B.Cu") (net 4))
 (segment (start 109.431 71.4785) (end 108.832 72.0775) (width 0.2) (layer "B.Cu") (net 4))
 (segment (start 108.832 82.416) (end 109.982 83.566) (width 0.2) (layer "B.Cu") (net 4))
 (segment (start 106.292 82.416) (end 107.442 83.566) (width 0.2) (layer "B.Cu") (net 6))
 (segment (start 106.661 71.4785) (end 106.292 71.8475) (width 0.2) (layer "B.Cu") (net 6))
 (segment (start 106.292 71.8475) (end 106.292 82.416) (width 0.2) (layer "B.Cu") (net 6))
 (segment (start 103.752 82.416) (end 104.902 83.566) (width 0.2) (layer "B.Cu") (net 8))
 (segment (start 103.752 71.6175) (end 103.752 82.416) (width 0.2) (layer "B.Cu") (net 8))
 (segment (start 103.891 71.4785) (end 103.752 71.6175) (width 0.2) (layer "B.Cu") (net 8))
 (segment (start 101.121 71.4785) (end 101.121 82.325) (width 0.2) (layer "B.Cu") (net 10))
 (segment (start 101.121 82.325) (end 102.362 83.566) (width 0.2) (layer "B.Cu") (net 10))
 (segment (start 98.672 71.7995) (end 98.672 82.416) (width 0.2) (layer "B.Cu") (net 12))
 (segment (start 98.672 82.416) (end 99.822 83.566) (width 0.2) (layer "B.Cu") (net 12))
 (segment (start 98.351 71.4785) (end 98.672 71.7995) (width 0.2) (layer "B.Cu") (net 12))
 (segment (start 95.892 71.7895) (end 95.892 82.176) (width 0.2) (layer "B.Cu") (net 13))
 (segment (start 95.892 82.176) (end 97.282 83.566) (width 0.2) (layer "B.Cu") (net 13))
 (segment (start 95.581 71.4785) (end 95.892 71.7895) (width 0.2) (layer "B.Cu") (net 13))
 (segment (start 93.592 82.416) (end 94.742 83.566) (width 0.2) (layer "B.Cu") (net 15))
 (segment (start 92.811 71.4785) (end 93.592 72.2595) (width 0.2) (layer "B.Cu") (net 15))
 (segment (start 93.592 72.2595) (end 93.592 82.416) (width 0.2) (layer "B.Cu") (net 15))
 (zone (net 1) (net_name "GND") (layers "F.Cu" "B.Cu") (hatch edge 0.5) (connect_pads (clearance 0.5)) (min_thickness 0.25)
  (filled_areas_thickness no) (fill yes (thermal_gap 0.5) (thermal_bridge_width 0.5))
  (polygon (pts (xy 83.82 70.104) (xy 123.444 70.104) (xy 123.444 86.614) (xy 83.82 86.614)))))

